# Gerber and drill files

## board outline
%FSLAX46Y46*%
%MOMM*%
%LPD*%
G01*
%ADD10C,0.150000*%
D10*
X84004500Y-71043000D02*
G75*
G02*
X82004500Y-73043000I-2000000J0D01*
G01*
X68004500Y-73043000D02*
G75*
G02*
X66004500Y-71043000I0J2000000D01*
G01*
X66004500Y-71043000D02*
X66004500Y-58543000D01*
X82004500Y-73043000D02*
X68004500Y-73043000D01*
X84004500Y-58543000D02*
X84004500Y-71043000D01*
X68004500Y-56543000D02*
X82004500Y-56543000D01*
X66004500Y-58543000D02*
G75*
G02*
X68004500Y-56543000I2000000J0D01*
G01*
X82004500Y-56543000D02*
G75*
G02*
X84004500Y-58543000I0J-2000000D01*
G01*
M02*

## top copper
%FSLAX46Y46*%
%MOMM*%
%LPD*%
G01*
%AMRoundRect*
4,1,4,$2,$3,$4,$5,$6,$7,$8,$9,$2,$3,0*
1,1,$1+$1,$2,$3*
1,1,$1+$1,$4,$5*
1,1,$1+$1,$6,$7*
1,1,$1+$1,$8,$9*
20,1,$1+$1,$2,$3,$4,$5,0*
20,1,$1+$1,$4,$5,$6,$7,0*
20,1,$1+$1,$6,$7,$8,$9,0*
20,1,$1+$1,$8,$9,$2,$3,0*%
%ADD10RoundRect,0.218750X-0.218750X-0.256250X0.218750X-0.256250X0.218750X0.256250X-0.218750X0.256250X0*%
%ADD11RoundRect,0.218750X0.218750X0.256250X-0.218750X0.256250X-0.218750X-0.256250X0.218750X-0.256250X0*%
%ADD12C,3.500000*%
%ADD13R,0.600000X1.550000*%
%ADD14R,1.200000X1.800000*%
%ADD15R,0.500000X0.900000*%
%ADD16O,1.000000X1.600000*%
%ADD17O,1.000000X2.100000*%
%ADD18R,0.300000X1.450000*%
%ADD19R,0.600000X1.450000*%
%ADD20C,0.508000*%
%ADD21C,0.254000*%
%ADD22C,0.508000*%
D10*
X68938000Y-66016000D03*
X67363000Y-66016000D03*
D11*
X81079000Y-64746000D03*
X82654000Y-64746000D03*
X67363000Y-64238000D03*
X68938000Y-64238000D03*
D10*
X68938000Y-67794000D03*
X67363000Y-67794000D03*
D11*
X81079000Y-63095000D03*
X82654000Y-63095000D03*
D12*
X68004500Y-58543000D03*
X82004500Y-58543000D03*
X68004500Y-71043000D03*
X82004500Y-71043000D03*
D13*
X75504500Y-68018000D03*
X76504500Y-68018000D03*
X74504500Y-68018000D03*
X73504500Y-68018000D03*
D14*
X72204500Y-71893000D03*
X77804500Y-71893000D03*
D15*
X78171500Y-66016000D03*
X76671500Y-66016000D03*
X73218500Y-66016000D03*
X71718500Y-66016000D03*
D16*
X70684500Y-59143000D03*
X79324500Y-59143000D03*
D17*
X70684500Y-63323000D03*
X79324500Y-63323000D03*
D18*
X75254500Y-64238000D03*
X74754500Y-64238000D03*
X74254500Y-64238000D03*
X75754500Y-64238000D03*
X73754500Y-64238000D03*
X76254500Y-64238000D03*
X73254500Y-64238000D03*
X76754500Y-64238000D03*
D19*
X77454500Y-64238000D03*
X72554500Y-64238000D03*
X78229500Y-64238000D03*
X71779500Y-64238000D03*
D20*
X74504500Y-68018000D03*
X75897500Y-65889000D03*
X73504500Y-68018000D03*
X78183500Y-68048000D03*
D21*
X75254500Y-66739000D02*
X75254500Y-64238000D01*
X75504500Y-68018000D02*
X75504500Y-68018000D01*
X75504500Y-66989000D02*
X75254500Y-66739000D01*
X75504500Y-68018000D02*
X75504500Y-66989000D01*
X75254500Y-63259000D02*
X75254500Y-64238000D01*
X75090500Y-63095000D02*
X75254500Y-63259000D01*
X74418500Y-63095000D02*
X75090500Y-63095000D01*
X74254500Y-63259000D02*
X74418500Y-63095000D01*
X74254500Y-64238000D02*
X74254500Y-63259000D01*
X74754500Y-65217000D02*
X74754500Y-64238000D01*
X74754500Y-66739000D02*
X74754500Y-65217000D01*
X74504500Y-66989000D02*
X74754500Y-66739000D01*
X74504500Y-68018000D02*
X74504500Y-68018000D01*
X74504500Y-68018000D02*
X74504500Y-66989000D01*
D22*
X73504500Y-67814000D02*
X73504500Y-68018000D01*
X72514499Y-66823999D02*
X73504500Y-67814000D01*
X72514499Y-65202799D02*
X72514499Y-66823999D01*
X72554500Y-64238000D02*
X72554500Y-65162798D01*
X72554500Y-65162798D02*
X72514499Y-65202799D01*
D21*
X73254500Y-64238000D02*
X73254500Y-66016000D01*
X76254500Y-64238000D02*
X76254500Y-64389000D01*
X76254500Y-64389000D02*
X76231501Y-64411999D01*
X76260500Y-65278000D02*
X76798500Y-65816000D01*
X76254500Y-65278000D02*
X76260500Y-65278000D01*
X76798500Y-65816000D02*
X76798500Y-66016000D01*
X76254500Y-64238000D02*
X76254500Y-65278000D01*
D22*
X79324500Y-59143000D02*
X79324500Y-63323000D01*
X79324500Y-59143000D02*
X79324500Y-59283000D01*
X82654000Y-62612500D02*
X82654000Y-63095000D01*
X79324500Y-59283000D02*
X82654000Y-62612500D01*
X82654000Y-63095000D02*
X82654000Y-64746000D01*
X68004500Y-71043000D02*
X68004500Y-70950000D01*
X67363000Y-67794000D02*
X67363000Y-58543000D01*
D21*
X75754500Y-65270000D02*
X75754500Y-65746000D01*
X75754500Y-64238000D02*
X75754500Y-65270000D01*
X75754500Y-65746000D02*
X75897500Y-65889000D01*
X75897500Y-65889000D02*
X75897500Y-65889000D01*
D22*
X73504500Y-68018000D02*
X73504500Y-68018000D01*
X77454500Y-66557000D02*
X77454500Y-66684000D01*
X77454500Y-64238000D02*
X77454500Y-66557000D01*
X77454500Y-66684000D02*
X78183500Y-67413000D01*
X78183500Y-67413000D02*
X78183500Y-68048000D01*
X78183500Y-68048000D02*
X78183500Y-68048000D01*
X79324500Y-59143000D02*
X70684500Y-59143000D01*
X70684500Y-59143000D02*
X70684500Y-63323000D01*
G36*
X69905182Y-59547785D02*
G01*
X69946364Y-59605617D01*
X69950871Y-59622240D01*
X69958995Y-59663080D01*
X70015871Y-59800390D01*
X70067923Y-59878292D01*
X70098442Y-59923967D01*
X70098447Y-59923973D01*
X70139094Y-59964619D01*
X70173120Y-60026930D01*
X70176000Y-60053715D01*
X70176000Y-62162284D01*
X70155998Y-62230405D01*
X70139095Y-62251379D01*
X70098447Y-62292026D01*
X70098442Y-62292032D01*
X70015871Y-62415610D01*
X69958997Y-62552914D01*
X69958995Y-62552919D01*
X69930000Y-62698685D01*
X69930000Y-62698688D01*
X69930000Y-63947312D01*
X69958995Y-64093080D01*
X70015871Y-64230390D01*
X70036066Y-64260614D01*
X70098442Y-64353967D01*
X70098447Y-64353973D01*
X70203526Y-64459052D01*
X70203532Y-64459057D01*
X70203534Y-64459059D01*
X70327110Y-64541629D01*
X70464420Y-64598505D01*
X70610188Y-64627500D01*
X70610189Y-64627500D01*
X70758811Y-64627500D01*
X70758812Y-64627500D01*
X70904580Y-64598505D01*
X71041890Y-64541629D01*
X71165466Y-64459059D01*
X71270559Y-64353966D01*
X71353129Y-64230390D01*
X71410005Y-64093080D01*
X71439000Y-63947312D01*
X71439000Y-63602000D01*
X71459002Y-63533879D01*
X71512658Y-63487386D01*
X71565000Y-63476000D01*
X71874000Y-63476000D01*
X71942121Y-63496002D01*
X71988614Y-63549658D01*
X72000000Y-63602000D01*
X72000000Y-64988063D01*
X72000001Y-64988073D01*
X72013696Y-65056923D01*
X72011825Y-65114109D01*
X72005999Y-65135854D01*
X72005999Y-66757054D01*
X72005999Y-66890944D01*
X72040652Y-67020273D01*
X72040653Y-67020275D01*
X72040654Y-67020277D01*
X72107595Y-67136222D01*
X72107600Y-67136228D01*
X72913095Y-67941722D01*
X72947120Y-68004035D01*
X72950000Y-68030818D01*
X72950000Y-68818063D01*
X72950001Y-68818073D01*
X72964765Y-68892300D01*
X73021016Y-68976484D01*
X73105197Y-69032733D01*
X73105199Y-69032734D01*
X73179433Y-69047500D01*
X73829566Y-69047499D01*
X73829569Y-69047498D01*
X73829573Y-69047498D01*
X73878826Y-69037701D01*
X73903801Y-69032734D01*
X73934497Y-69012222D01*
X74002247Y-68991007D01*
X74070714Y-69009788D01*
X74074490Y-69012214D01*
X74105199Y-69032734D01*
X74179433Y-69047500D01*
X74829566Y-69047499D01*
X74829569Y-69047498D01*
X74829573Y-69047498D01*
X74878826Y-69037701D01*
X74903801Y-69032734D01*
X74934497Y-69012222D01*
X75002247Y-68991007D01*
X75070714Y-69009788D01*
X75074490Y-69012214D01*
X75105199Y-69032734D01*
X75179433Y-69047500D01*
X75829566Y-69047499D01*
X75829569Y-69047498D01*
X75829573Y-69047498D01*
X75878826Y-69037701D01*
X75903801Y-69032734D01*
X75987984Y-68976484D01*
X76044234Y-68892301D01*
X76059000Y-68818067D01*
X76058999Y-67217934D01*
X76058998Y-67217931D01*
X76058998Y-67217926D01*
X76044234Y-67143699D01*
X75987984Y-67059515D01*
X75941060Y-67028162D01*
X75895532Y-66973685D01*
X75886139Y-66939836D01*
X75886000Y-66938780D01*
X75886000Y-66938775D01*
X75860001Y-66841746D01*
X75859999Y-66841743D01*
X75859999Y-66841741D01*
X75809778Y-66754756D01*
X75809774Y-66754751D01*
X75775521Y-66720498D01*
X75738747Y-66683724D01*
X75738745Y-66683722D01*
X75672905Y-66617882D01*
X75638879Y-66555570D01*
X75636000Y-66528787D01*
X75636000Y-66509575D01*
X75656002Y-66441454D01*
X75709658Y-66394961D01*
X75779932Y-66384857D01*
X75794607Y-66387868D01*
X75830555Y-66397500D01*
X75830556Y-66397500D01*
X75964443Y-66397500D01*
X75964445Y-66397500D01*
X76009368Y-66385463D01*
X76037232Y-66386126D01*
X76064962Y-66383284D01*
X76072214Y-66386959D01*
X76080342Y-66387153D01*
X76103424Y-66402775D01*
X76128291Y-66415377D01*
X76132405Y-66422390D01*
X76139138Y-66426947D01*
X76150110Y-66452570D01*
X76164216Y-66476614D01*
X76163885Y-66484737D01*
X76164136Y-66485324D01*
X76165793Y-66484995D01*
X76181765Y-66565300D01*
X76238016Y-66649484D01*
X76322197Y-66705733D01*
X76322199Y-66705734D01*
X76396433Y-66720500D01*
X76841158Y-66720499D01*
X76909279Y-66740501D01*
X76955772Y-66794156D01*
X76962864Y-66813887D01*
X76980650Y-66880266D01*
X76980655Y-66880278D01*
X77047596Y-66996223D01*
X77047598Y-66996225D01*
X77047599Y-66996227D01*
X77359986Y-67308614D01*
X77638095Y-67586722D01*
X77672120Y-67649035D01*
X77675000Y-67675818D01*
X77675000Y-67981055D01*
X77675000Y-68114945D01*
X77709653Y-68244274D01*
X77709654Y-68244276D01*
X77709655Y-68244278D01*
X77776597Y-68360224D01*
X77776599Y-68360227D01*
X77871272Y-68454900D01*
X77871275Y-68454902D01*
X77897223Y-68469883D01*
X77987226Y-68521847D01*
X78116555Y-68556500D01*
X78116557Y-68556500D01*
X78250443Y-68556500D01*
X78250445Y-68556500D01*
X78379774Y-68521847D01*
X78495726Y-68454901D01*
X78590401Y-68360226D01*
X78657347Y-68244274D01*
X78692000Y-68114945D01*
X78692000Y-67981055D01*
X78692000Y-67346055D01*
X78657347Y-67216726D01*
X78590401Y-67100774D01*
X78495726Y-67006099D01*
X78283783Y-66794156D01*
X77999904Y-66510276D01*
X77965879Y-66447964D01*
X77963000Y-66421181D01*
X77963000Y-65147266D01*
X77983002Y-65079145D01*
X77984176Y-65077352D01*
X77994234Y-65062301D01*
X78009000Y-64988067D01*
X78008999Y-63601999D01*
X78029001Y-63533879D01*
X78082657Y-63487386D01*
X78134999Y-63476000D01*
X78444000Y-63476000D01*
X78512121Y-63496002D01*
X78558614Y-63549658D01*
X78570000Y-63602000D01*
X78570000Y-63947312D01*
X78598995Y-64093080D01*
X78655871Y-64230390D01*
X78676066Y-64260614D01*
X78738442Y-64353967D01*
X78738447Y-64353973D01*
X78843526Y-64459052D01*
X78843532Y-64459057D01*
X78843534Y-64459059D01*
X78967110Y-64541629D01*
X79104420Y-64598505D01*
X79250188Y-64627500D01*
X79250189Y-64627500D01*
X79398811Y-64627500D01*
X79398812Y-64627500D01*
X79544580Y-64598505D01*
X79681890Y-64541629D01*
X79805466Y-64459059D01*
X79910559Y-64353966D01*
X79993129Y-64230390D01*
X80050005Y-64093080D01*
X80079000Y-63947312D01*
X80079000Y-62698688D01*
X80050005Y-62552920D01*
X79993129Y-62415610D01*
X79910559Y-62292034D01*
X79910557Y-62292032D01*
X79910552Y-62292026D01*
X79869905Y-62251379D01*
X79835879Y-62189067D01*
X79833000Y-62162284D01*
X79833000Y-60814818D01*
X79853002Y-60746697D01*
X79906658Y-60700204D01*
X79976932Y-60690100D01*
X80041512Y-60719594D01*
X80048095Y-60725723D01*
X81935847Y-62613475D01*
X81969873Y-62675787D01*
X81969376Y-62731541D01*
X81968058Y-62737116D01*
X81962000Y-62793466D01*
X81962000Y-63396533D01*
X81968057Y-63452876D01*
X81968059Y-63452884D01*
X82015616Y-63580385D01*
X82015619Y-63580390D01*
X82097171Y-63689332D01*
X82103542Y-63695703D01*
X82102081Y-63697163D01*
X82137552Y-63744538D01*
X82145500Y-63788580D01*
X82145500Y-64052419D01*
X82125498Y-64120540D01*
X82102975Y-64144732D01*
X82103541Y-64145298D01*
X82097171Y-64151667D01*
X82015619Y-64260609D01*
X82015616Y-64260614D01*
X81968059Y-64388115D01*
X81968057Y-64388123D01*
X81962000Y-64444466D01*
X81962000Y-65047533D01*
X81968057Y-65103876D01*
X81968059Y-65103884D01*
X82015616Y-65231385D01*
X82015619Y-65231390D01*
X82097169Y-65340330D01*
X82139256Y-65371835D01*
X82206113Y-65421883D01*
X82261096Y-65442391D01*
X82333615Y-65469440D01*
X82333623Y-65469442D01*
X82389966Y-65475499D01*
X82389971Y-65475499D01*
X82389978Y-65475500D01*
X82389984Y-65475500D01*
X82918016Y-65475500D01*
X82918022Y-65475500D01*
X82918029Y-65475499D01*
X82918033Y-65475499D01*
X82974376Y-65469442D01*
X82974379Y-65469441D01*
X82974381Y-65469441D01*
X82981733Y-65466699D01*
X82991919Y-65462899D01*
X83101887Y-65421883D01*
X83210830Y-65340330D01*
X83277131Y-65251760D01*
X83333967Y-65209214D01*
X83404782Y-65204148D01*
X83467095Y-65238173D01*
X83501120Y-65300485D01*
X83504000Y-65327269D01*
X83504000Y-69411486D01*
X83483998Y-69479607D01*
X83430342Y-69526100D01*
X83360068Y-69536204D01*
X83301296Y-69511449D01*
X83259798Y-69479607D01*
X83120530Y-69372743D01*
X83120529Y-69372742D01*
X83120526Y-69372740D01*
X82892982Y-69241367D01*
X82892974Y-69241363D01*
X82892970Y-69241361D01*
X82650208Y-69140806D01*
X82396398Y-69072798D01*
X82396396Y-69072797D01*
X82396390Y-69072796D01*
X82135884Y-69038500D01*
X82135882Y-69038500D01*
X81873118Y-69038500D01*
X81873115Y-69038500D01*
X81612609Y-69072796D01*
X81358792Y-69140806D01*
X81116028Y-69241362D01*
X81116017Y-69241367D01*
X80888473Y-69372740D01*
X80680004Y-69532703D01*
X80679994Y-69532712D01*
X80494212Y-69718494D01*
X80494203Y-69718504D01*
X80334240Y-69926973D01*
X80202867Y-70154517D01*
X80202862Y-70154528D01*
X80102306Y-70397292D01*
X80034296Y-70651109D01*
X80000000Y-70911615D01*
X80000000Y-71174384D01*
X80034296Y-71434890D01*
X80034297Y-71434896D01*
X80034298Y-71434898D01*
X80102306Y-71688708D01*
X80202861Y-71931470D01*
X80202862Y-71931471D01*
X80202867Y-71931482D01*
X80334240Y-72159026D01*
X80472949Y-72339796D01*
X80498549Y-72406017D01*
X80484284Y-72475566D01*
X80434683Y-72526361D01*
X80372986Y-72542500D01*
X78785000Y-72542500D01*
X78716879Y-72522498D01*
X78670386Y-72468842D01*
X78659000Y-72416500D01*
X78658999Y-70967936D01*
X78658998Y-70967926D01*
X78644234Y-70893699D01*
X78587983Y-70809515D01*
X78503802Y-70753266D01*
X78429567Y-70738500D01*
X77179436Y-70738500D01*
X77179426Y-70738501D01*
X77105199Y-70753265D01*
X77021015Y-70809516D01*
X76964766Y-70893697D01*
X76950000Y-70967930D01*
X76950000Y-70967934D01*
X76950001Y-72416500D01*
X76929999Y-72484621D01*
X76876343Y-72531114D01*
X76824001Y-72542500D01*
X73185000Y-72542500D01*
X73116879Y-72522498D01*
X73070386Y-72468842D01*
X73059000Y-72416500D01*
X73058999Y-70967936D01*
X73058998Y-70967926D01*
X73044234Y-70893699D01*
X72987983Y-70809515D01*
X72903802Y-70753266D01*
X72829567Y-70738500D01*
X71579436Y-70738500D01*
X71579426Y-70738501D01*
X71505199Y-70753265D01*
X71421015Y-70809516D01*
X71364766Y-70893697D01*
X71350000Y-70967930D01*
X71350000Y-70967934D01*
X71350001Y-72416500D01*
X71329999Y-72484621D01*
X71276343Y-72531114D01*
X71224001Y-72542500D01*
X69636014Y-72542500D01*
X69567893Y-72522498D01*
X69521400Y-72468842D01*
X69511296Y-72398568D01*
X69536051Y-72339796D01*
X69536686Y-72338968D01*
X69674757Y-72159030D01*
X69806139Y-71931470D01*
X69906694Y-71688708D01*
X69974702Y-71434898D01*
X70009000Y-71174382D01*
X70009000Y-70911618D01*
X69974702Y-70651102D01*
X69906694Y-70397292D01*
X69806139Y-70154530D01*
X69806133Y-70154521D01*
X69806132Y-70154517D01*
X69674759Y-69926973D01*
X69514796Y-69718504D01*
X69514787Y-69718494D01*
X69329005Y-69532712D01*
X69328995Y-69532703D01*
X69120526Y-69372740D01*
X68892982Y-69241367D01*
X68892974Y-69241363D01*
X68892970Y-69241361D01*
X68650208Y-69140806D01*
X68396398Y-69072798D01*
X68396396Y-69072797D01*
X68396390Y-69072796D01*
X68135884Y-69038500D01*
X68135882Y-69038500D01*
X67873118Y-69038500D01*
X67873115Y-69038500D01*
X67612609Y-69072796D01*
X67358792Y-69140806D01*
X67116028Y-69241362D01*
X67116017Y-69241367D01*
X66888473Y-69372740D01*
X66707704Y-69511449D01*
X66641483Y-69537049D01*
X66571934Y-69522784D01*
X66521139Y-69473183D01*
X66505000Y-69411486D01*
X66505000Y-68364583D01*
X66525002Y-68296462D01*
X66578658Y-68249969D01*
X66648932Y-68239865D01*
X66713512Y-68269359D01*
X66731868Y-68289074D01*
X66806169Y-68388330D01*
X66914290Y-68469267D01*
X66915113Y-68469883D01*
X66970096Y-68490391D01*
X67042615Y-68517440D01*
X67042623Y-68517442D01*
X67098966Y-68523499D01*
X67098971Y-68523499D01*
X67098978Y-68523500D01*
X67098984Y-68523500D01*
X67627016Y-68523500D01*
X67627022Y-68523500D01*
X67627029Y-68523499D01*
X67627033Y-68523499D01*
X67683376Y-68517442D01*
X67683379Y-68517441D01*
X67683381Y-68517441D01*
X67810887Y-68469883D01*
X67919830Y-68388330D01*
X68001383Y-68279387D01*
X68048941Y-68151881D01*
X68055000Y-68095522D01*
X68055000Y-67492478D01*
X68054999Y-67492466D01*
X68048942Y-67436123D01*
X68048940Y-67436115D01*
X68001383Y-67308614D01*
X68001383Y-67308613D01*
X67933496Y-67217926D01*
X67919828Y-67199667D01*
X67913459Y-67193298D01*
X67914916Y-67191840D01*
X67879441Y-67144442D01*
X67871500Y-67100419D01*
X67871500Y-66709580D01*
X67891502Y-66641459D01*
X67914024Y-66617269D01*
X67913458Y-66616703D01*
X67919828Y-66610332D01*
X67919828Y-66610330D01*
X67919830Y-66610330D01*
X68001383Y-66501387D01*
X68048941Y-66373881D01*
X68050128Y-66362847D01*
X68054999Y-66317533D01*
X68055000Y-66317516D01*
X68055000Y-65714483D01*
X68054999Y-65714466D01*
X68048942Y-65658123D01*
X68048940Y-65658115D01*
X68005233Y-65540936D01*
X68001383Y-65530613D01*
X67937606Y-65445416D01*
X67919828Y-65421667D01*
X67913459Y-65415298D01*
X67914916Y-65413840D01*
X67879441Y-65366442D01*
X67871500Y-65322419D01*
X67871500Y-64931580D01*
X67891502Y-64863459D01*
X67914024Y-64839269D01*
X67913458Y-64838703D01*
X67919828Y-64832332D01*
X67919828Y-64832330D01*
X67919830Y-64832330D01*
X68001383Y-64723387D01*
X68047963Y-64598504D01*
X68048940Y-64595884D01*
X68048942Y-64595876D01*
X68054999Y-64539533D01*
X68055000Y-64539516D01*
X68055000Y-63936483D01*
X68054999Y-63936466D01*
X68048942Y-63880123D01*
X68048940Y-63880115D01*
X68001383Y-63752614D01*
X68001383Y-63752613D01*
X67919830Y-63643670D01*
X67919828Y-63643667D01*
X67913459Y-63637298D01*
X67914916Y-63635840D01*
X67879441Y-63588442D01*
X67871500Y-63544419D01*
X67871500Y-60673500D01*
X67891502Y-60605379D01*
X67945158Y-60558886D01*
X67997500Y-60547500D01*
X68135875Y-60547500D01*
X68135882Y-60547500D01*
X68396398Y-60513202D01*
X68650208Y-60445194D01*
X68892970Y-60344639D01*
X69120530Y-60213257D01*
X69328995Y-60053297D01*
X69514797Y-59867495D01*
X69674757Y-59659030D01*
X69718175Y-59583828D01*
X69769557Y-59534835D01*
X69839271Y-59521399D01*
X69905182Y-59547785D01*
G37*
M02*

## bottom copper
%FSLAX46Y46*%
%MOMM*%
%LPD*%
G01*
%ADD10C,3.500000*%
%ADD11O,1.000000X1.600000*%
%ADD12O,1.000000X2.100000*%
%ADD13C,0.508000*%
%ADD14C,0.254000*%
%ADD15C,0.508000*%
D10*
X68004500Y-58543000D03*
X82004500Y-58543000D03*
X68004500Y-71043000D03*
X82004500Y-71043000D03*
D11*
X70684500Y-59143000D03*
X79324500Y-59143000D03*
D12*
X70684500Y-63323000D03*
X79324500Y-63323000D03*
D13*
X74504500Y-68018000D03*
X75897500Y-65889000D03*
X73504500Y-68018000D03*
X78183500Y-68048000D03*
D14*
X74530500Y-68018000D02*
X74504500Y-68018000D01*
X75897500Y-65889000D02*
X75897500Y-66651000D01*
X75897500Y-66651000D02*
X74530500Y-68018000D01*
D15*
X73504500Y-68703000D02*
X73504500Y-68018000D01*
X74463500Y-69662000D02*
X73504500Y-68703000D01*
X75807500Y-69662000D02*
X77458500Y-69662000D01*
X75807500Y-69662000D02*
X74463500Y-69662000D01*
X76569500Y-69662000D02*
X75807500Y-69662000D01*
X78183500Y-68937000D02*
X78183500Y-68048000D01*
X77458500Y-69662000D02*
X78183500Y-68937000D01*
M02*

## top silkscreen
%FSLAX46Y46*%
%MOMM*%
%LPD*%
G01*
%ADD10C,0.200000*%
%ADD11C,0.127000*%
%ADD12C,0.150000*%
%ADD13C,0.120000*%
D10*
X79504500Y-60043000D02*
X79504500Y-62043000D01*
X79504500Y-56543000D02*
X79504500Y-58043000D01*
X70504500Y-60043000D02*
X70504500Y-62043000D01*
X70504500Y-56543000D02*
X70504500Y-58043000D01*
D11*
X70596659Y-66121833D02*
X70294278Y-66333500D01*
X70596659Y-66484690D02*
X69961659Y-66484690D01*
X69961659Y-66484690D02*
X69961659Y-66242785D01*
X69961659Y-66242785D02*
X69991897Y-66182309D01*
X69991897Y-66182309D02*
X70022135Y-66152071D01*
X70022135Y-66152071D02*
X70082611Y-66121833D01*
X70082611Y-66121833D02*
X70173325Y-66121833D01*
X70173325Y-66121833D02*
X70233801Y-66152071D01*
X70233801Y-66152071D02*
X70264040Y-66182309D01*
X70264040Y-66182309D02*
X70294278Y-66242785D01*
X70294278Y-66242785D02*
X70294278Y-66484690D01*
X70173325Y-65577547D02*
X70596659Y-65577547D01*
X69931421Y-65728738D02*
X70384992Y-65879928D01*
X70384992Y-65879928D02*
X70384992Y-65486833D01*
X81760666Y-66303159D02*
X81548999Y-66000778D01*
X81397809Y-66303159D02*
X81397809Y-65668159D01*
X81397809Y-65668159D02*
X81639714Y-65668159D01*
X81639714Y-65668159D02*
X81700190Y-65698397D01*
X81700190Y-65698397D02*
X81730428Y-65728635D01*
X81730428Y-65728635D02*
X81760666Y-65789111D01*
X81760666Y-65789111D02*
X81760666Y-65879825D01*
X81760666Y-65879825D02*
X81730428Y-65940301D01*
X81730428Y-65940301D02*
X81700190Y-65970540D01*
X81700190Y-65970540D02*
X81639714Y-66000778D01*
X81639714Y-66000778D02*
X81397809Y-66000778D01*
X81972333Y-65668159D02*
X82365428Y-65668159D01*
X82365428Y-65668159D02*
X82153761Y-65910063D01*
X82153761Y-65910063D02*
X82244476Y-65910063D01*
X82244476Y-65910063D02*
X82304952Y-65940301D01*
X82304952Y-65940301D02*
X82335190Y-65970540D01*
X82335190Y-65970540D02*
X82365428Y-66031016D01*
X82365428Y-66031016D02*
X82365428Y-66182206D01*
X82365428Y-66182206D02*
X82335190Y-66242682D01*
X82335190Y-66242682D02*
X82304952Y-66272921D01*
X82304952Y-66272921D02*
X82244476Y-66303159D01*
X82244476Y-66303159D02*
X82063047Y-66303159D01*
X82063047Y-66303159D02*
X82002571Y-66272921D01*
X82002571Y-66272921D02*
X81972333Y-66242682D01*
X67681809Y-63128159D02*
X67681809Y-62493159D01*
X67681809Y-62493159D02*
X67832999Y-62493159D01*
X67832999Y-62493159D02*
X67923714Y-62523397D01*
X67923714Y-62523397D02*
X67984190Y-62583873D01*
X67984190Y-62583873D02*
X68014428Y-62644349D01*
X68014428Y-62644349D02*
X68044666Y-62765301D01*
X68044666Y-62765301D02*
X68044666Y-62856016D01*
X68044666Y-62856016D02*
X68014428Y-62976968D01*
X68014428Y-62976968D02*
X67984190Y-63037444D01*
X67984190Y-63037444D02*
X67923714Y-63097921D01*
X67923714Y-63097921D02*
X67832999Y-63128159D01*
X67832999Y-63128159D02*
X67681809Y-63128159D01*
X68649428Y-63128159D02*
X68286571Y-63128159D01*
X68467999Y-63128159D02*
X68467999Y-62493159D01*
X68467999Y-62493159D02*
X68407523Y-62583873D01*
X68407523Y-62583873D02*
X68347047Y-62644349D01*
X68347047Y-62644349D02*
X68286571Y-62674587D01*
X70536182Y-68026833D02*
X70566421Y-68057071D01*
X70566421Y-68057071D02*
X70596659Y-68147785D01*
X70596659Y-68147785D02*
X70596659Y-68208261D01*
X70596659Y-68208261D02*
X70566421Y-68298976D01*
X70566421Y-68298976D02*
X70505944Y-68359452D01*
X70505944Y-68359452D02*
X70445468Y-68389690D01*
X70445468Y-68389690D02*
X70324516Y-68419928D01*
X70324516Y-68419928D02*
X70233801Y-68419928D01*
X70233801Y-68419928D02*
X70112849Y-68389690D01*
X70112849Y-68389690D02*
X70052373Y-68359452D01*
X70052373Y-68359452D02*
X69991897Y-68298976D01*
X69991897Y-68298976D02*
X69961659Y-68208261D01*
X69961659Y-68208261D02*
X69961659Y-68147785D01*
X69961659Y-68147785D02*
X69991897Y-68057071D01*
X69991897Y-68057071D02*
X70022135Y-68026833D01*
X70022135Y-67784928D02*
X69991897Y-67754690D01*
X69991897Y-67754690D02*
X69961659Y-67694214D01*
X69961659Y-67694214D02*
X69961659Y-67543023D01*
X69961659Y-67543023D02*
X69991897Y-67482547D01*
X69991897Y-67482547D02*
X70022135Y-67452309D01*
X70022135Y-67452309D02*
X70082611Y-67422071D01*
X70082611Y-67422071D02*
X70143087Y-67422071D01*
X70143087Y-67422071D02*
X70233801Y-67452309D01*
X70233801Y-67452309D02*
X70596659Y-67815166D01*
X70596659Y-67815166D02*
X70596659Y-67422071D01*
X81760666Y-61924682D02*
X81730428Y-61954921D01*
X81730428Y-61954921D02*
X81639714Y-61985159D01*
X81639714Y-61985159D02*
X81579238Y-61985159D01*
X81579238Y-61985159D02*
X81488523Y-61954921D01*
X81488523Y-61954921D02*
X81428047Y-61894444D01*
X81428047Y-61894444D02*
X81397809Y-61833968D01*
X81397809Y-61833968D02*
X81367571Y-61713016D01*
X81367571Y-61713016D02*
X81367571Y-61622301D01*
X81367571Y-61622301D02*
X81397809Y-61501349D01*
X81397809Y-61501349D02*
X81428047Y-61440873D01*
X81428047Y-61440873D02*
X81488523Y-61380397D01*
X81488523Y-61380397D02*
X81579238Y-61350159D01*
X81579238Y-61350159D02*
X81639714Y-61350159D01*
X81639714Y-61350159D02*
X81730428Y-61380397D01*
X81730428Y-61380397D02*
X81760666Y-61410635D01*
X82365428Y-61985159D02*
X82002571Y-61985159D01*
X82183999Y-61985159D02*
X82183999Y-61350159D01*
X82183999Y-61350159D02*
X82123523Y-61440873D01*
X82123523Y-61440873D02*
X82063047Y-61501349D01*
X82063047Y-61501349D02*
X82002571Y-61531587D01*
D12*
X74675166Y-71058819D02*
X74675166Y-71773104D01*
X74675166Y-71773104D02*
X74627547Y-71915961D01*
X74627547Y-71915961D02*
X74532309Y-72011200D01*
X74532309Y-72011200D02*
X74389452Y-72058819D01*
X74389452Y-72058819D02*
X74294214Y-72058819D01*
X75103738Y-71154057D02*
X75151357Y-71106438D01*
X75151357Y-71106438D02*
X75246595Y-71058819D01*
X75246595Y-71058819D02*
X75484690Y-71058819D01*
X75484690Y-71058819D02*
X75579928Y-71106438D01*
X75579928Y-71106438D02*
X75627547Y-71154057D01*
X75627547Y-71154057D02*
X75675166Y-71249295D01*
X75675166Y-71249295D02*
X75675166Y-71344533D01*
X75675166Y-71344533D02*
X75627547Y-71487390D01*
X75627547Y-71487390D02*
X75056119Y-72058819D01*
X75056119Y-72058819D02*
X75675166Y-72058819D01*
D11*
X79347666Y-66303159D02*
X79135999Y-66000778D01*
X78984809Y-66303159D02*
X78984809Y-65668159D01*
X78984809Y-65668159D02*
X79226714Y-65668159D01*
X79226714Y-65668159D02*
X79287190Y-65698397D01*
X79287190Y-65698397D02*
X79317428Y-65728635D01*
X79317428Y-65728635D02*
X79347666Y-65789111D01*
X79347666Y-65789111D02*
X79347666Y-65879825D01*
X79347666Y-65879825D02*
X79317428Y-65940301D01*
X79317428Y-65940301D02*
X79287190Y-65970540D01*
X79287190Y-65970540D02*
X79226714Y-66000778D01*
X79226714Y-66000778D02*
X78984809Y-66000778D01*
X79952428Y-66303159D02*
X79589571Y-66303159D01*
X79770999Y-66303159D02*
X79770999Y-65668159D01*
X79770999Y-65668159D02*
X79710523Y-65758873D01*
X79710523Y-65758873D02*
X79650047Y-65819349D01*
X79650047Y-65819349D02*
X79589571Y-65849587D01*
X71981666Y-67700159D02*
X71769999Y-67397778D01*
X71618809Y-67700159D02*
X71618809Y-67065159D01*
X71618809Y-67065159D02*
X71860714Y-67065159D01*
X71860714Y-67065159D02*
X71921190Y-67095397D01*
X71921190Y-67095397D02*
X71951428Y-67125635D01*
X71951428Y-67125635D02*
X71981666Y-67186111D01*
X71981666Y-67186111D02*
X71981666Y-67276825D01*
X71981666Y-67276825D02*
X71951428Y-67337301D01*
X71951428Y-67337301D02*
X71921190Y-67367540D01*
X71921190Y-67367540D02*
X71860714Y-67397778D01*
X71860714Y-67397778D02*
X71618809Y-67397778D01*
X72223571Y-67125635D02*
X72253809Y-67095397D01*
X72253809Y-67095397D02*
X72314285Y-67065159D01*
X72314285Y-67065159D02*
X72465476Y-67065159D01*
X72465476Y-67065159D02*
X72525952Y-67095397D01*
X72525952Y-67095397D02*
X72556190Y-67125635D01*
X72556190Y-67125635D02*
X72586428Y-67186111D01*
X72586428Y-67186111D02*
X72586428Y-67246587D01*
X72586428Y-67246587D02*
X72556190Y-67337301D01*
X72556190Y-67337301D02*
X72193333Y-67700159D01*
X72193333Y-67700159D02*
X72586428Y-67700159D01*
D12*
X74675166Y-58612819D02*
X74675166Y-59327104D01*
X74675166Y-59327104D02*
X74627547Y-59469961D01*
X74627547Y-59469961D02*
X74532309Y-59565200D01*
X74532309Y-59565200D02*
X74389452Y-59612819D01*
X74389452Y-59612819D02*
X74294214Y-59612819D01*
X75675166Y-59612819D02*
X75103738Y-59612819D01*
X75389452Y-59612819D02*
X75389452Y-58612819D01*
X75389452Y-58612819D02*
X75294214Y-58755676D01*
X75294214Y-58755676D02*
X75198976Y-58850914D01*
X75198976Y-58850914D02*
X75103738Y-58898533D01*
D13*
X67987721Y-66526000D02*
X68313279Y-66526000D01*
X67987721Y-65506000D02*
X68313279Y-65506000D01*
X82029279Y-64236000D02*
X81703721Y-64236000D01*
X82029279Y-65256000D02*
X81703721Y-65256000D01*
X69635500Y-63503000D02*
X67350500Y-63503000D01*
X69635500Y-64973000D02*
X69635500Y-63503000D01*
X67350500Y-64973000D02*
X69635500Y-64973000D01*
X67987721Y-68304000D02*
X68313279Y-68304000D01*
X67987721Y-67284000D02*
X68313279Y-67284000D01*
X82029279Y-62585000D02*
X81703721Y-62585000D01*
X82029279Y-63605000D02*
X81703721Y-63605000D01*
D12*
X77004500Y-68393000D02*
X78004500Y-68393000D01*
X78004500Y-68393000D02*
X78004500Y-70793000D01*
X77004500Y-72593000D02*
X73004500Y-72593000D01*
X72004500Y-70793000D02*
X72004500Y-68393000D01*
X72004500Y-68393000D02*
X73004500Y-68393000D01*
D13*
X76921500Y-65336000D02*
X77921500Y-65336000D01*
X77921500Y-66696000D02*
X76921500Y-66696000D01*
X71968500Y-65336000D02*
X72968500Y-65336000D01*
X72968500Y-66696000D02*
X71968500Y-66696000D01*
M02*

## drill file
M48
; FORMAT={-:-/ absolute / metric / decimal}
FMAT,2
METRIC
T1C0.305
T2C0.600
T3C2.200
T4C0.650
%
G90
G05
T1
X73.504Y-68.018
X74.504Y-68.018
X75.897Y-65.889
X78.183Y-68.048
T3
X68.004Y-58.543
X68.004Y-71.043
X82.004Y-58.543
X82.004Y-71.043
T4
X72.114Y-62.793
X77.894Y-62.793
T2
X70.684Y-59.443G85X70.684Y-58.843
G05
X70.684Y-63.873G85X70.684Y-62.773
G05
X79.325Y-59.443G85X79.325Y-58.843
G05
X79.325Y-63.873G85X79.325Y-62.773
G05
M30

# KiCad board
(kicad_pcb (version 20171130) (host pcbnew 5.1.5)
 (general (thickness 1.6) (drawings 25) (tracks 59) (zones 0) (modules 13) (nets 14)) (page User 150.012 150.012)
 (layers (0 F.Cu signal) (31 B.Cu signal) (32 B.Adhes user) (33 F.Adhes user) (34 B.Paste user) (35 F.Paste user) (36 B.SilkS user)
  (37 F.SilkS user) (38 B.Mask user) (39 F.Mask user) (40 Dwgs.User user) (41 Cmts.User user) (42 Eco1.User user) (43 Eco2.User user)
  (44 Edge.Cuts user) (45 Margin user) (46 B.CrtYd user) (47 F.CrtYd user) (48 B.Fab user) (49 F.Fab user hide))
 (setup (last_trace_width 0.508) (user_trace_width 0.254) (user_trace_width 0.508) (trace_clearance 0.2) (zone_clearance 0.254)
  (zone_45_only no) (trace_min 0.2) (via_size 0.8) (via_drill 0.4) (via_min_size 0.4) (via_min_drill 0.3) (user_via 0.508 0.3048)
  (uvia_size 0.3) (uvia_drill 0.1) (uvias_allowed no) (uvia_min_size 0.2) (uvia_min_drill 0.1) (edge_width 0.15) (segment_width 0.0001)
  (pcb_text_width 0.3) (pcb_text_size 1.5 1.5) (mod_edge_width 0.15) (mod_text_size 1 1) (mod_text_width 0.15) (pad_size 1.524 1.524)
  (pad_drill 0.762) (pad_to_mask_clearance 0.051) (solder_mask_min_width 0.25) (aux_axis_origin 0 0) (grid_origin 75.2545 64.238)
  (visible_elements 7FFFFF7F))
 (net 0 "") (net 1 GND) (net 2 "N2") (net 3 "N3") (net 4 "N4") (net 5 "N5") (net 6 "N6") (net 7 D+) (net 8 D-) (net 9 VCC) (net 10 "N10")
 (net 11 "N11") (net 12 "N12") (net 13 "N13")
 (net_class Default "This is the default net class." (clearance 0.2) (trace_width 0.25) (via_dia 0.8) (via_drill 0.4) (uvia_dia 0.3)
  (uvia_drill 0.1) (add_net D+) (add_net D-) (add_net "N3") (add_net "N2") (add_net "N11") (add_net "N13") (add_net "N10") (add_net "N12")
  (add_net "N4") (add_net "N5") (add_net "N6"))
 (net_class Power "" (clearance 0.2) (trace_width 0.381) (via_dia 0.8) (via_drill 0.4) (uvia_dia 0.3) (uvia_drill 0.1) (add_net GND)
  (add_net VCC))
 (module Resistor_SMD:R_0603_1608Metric (layer F.Cu) (at 68.1505 66.016)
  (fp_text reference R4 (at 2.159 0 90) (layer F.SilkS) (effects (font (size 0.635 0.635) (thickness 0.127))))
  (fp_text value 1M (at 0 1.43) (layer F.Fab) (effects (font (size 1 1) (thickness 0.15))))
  (fp_line (start -0.162779 0.51) (end 0.162779 0.51) (layer F.SilkS) (width 0.12))
  (fp_line (start -0.162779 -0.51) (end 0.162779 -0.51) (layer F.SilkS) (width 0.12))
  (pad 2 smd roundrect (at 0.7875 0) (size 0.875 0.95) (layers F.Cu F.Paste F.Mask) (roundrect_rratio 0.25) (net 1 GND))
  (pad 1 smd roundrect (at -0.7875 0) (size 0.875 0.95) (layers F.Cu F.Paste F.Mask) (roundrect_rratio 0.25) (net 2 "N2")))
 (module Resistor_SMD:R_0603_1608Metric (layer F.Cu) (at 81.8665 64.746 180)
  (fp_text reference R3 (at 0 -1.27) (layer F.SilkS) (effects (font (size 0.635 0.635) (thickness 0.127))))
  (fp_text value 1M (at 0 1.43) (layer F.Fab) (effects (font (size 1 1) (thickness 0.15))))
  (fp_line (start -0.162779 0.51) (end 0.162779 0.51) (layer F.SilkS) (width 0.12))
  (fp_line (start -0.162779 -0.51) (end 0.162779 -0.51) (layer F.SilkS) (width 0.12))
  (pad 2 smd roundrect (at 0.7875 0 180) (size 0.875 0.95) (layers F.Cu F.Paste F.Mask) (roundrect_rratio 0.25) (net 1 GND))
  (pad 1 smd roundrect (at -0.7875 0 180) (size 0.875 0.95) (layers F.Cu F.Paste F.Mask) (roundrect_rratio 0.25) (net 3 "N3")))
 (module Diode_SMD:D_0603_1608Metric (layer F.Cu) (at 68.1505 64.238 180)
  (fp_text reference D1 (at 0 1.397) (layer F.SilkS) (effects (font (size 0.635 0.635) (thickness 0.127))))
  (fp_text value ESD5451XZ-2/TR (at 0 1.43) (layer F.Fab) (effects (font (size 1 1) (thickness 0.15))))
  (fp_line (start -1.485 0.735) (end 0.8 0.735) (layer F.SilkS) (width 0.12))
  (fp_line (start -1.485 -0.735) (end -1.485 0.735) (layer F.SilkS) (width 0.12))
  (fp_line (start 0.8 -0.735) (end -1.485 -0.735) (layer F.SilkS) (width 0.12))
  (pad 2 smd roundrect (at 0.7875 0 180) (size 0.875 0.95) (layers F.Cu F.Paste F.Mask) (roundrect_rratio 0.25) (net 2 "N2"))
  (pad 1 smd roundrect (at -0.7875 0 180) (size 0.875 0.95) (layers F.Cu F.Paste F.Mask) (roundrect_rratio 0.25) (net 1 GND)))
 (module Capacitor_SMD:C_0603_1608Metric (layer F.Cu) (at 68.1505 67.794)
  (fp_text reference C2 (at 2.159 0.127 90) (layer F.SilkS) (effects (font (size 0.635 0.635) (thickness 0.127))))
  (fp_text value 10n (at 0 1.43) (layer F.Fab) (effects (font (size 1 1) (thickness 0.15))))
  (fp_line (start -0.162779 0.51) (end 0.162779 0.51) (layer F.SilkS) (width 0.12))
  (fp_line (start -0.162779 -0.51) (end 0.162779 -0.51) (layer F.SilkS) (width 0.12))
  (pad 2 smd roundrect (at 0.7875 0) (size 0.875 0.95) (layers F.Cu F.Paste F.Mask) (roundrect_rratio 0.25) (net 1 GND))
  (pad 1 smd roundrect (at -0.7875 0) (size 0.875 0.95) (layers F.Cu F.Paste F.Mask) (roundrect_rratio 0.25) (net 2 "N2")))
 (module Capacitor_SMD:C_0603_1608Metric (layer F.Cu) (at 81.8665 63.095 180)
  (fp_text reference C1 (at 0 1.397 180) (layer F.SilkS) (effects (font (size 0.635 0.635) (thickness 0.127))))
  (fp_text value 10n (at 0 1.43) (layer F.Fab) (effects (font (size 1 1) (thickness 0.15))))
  (fp_line (start -0.162779 0.51) (end 0.162779 0.51) (layer F.SilkS) (width 0.12))
  (fp_line (start -0.162779 -0.51) (end 0.162779 -0.51) (layer F.SilkS) (width 0.12))
  (pad 2 smd roundrect (at 0.7875 0 180) (size 0.875 0.95) (layers F.Cu F.Paste F.Mask) (roundrect_rratio 0.25) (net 1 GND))
  (pad 1 smd roundrect (at -0.7875 0 180) (size 0.875 0.95) (layers F.Cu F.Paste F.Mask) (roundrect_rratio 0.25) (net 3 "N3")))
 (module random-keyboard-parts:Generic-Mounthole (layer F.Cu) (at 68.0045 58.543)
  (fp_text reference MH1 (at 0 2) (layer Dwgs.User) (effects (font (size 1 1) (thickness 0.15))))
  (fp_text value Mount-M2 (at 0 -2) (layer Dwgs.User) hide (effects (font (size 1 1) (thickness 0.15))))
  (pad 1 thru_hole circle (at 0 0) (size 3.5 3.5) (drill 2.2) (layers *.Cu *.Mask) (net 2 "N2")))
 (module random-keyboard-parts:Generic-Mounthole (layer F.Cu) (at 82.0045 58.543)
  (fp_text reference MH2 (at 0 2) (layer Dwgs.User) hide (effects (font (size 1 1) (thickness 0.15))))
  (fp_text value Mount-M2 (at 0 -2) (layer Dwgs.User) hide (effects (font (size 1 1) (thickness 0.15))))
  (pad 1 thru_hole circle (at 0 0) (size 3.5 3.5) (drill 2.2) (layers *.Cu *.Mask) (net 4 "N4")))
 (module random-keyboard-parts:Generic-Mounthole (layer F.Cu) (at 68.0045 71.043)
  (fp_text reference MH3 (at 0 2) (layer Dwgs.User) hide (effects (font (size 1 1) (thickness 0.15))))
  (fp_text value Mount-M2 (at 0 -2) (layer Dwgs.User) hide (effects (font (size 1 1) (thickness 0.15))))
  (pad 1 thru_hole circle (at 0 0) (size 3.5 3.5) (drill 2.2) (layers *.Cu *.Mask) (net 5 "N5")))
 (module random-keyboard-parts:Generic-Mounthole (layer F.Cu) (at 82.0045 71.043)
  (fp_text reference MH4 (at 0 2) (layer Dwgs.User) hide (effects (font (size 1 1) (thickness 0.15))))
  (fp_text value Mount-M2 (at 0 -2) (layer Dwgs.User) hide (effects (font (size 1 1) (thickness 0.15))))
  (pad 1 thru_hole circle (at 0 0) (size 3.5 3.5) (drill 2.2) (layers *.Cu *.Mask) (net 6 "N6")))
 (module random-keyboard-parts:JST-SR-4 (layer F.Cu) (at 75.0045 72.793)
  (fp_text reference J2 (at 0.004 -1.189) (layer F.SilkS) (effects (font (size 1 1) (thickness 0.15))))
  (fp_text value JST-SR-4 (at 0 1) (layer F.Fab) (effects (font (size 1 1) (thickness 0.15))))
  (fp_line (start 2 -4.4) (end 3 -4.4) (layer F.SilkS) (width 0.15))
  (fp_line (start 3 -4.4) (end 3 -2) (layer F.SilkS) (width 0.15))
  (fp_line (start 2 -0.2) (end -2 -0.2) (layer F.SilkS) (width 0.15))
  (fp_line (start -3 -2) (end -3 -4.4) (layer F.SilkS) (width 0.15))
  (fp_line (start -3 -4.4) (end -2 -4.4) (layer F.SilkS) (width 0.15))
  (pad 3 smd rect (at 0.5 -4.775) (size 0.6 1.55) (layers F.Cu F.Paste F.Mask) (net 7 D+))
  (pad 4 smd rect (at 1.5 -4.775) (size 0.6 1.55) (layers F.Cu F.Paste F.Mask) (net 1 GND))
  (pad 2 smd rect (at -0.5 -4.775) (size 0.6 1.55) (layers F.Cu F.Paste F.Mask) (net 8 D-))
  (pad 1 smd rect (at -1.5 -4.775) (size 0.6 1.55) (layers F.Cu F.Paste F.Mask) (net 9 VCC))
  (pad "" smd rect (at -2.8 -0.9) (size 1.2 1.8) (layers F.Cu F.Paste F.Mask))
  (pad "" smd rect (at 2.8 -0.9) (size 1.2 1.8) (layers F.Cu F.Paste F.Mask)))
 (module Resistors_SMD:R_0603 (layer F.Cu) (at 77.4215 66.016)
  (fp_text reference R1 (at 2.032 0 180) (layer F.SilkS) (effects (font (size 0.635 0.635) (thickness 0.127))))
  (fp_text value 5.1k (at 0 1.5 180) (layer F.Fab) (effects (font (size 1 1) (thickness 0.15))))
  (fp_line (start -0.5 -0.68) (end 0.5 -0.68) (layer F.SilkS) (width 0.12))
  (fp_line (start 0.5 0.68) (end -0.5 0.68) (layer F.SilkS) (width 0.12))
  (pad 2 smd rect (at 0.75 0) (size 0.5 0.9) (layers F.Cu F.Paste F.Mask) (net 1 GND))
  (pad 1 smd rect (at -0.75 0) (size 0.5 0.9) (layers F.Cu F.Paste F.Mask) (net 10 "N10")))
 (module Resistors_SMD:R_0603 (layer F.Cu) (at 72.4685 66.016 180)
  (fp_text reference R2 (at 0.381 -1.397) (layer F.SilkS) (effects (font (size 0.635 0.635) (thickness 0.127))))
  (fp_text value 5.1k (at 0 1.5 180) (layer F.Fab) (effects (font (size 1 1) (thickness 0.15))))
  (fp_line (start 0.5 0.68) (end -0.5 0.68) (layer F.SilkS) (width 0.12))
  (fp_line (start -0.5 -0.68) (end 0.5 -0.68) (layer F.SilkS) (width 0.12))
  (pad 1 smd rect (at -0.75 0 180) (size 0.5 0.9) (layers F.Cu F.Paste F.Mask) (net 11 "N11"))
  (pad 2 smd rect (at 0.75 0 180) (size 0.5 0.9) (layers F.Cu F.Paste F.Mask) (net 1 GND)))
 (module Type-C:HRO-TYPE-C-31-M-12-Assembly (layer F.Cu) (at 75.0045 56.543 180)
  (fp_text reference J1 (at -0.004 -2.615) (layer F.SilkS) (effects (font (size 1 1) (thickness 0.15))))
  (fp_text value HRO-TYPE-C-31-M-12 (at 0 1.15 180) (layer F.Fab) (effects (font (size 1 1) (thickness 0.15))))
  (pad 13 thru_hole oval (at 4.32 -2.6 180) (size 1 1.6) (drill oval 0.6 1.2) (layers *.Cu *.Mask) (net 3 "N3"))
  (pad 13 thru_hole oval (at -4.32 -2.6 180) (size 1 1.6) (drill oval 0.6 1.2) (layers *.Cu *.Mask) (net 3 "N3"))
  (pad 13 thru_hole oval (at 4.32 -6.78 180) (size 1 2.1) (drill oval 0.6 1.7) (layers *.Cu *.Mask) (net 3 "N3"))
  (pad 13 thru_hole oval (at -4.32 -6.78 180) (size 1 2.1) (drill oval 0.6 1.7) (layers *.Cu *.Mask) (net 3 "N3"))
  (pad "" np_thru_hole circle (at -2.89 -6.25 180) (size 0.65 0.65) (drill 0.65) (layers *.Cu *.Mask))
  (pad "" np_thru_hole circle (at 2.89 -6.25 180) (size 0.65 0.65) (drill 0.65) (layers *.Cu *.Mask))
  (pad 6 smd rect (at -0.25 -7.695 180) (size 0.3 1.45) (layers F.Cu F.Paste F.Mask) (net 7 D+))
  (pad 7 smd rect (at 0.25 -7.695 180) (size 0.3 1.45) (layers F.Cu F.Paste F.Mask) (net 8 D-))
  (pad 8 smd rect (at 0.75 -7.695 180) (size 0.3 1.45) (layers F.Cu F.Paste F.Mask) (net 7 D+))
  (pad 5 smd rect (at -0.75 -7.695 180) (size 0.3 1.45) (layers F.Cu F.Paste F.Mask) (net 8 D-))
  (pad 9 smd rect (at 1.25 -7.695 180) (size 0.3 1.45) (layers F.Cu F.Paste F.Mask) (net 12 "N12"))
  (pad 4 smd rect (at -1.25 -7.695 180) (size 0.3 1.45) (layers F.Cu F.Paste F.Mask) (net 10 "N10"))
  (pad 10 smd rect (at 1.75 -7.695 180) (size 0.3 1.45) (layers F.Cu F.Paste F.Mask) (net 11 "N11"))
  (pad 3 smd rect (at -1.75 -7.695 180) (size 0.3 1.45) (layers F.Cu F.Paste F.Mask) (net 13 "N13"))
  (pad 2 smd rect (at -2.45 -7.695 180) (size 0.6 1.45) (layers F.Cu F.Paste F.Mask) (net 9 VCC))
  (pad 11 smd rect (at 2.45 -7.695 180) (size 0.6 1.45) (layers F.Cu F.Paste F.Mask) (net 9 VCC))
  (pad 1 smd rect (at -3.225 -7.695 180) (size 0.6 1.45) (layers F.Cu F.Paste F.Mask) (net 1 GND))
  (pad 12 smd rect (at 3.225 -7.695 180) (size 0.6 1.45) (layers F.Cu F.Paste F.Mask) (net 1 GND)))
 (gr_line (start 79.5045 60.043) (end 79.5045 62.043) (layer F.SilkS) (width 0.2))
 (gr_line (start 79.5045 56.543) (end 79.5045 58.043) (layer F.SilkS) (width 0.2))
 (gr_line (start 70.5045 60.043) (end 70.5045 62.043) (layer F.SilkS) (width 0.2))
 (gr_line (start 70.5045 56.543) (end 70.5045 58.043) (layer F.SilkS) (width 0.2))
 (gr_arc (start 82.0045 71.043) (end 82.0045 73.043) (angle -90) (layer Edge.Cuts) (width 0.15))
 (gr_arc (start 68.0045 71.043) (end 66.0045 71.043) (angle -90) (layer Edge.Cuts) (width 0.15))
 (gr_line (start 66.0045 71.043) (end 66.0045 58.543) (layer Edge.Cuts) (width 0.15))
 (gr_line (start 82.0045 73.043) (end 68.0045 73.043) (layer Edge.Cuts) (width 0.15))
 (gr_line (start 84.0045 58.543) (end 84.0045 71.043) (layer Edge.Cuts) (width 0.15))
 (gr_line (start 68.0045 56.543) (end 82.0045 56.543) (layer Edge.Cuts) (width 0.15))
 (gr_arc (start 68.0045 58.543) (end 68.0045 56.543) (angle -90) (layer Edge.Cuts) (width 0.15))
 (gr_arc (start 82.0045 58.543) (end 84.0045 58.543) (angle -90) (layer Edge.Cuts) (width 0.15))
 (segment (start 75.2545 66.739) (end 75.2545 64.238) (width 0.254) (layer F.Cu) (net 7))
 (segment (start 75.5045 68.018) (end 75.5045 68.018) (width 0.254) (layer F.Cu) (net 7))
 (segment (start 75.5045 66.989) (end 75.2545 66.739) (width 0.254) (layer F.Cu) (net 7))
 (segment (start 75.5045 68.018) (end 75.5045 66.989) (width 0.254) (layer F.Cu) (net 7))
 (segment (start 75.2545 63.259) (end 75.2545 64.238) (width 0.254) (layer F.Cu) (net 7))
 (segment (start 75.0905 63.095) (end 75.2545 63.259) (width 0.254) (layer F.Cu) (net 7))
 (segment (start 74.4185 63.095) (end 75.0905 63.095) (width 0.254) (layer F.Cu) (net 7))
 (segment (start 74.2545 63.259) (end 74.4185 63.095) (width 0.254) (layer F.Cu) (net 7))
 (segment (start 74.2545 64.238) (end 74.2545 63.259) (width 0.254) (layer F.Cu) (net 7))
 (segment (start 74.7545 65.217) (end 74.7545 64.238) (width 0.254) (layer F.Cu) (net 8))
 (segment (start 74.7545 66.739) (end 74.7545 65.217) (width 0.254) (layer F.Cu) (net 8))
 (segment (start 74.5045 66.989) (end 74.7545 66.739) (width 0.254) (layer F.Cu) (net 8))
 (segment (start 74.5045 68.018) (end 74.5045 68.018) (width 0.254) (layer F.Cu) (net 8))
 (segment (start 74.5045 68.018) (end 74.5045 66.989) (width 0.254) (layer F.Cu) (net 8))
 (via (at 74.5045 68.018) (size 0.508) (drill 0.3048) (layers F.Cu B.Cu) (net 8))
 (segment (start 73.5045 67.814) (end 73.5045 68.018) (width 0.508) (layer F.Cu) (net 9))
 (segment (start 72.514499 66.823999) (end 73.5045 67.814) (width 0.508) (layer F.Cu) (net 9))
 (segment (start 72.514499 65.202799) (end 72.514499 66.823999) (width 0.508) (layer F.Cu) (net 9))
 (segment (start 72.5545 64.238) (end 72.5545 65.162798) (width 0.508) (layer F.Cu) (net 9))
 (segment (start 72.5545 65.162798) (end 72.514499 65.202799) (width 0.508) (layer F.Cu) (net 9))
 (segment (start 73.2545 64.238) (end 73.2545 66.016) (width 0.254) (layer F.Cu) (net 11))
 (segment (start 76.2545 64.238) (end 76.2545 64.389) (width 0.254) (layer F.Cu) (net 10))
 (segment (start 76.2545 64.389) (end 76.231501 64.411999) (width 0.254) (layer F.Cu) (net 10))
 (segment (start 76.2605 65.278) (end 76.7985 65.816) (width 0.254) (layer F.Cu) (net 10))
 (segment (start 76.2545 65.278) (end 76.2605 65.278) (width 0.254) (layer F.Cu) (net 10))
 (segment (start 76.7985 65.816) (end 76.7985 66.016) (width 0.254) (layer F.Cu) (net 10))
 (segment (start 76.2545 64.238) (end 76.2545 65.278) (width 0.254) (layer F.Cu) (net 10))
 (segment (start 79.3245 59.143) (end 79.3245 63.323) (width 0.508) (layer F.Cu) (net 3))
 (segment (start 79.3245 59.143) (end 79.3245 59.283) (width 0.508) (layer F.Cu) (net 3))
 (segment (start 82.654 62.6125) (end 82.654 63.095) (width 0.508) (layer F.Cu) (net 3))
 (segment (start 79.3245 59.283) (end 82.654 62.6125) (width 0.508) (layer F.Cu) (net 3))
 (segment (start 82.654 63.095) (end 82.654 64.746) (width 0.508) (layer F.Cu) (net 3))
 (segment (start 68.0045 71.043) (end 68.0045 70.95) (width 0.508) (layer F.Cu) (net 5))
 (segment (start 67.363 67.794) (end 67.363 58.543) (width 0.508) (layer F.Cu) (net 2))
 (segment (start 75.7545 65.27) (end 75.7545 65.746) (width 0.254) (layer F.Cu) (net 8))
 (segment (start 75.7545 64.238) (end 75.7545 65.27) (width 0.254) (layer F.Cu) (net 8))
 (segment (start 75.7545 65.746) (end 75.8975 65.889) (width 0.254) (layer F.Cu) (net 8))
 (segment (start 75.8975 65.889) (end 75.8975 65.889) (width 0.254) (layer F.Cu) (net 8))
 (via (at 75.8975 65.889) (size 0.508) (drill 0.3048) (layers F.Cu B.Cu) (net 8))
 (segment (start 74.5305 68.018) (end 74.5045 68.018) (width 0.254) (layer B.Cu) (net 8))
 (segment (start 75.8975 65.889) (end 75.8975 66.651) (width 0.254) (layer B.Cu) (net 8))
 (segment (start 75.8975 66.651) (end 74.5305 68.018) (width 0.254) (layer B.Cu) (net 8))
 (segment (start 73.5045 68.018) (end 73.5045 68.018) (width 0.508) (layer F.Cu) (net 9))
 (via (at 73.5045 68.018) (size 0.508) (drill 0.3048) (layers F.Cu B.Cu) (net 9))
 (segment (start 73.5045 68.703) (end 73.5045 68.018) (width 0.508) (layer B.Cu) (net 9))
 (segment (start 74.4635 69.662) (end 73.5045 68.703) (width 0.508) (layer B.Cu) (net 9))
 (segment (start 77.4545 66.557) (end 77.4545 66.684) (width 0.508) (layer F.Cu) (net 9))
 (segment (start 77.4545 64.238) (end 77.4545 66.557) (width 0.508) (layer F.Cu) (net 9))
 (segment (start 77.4545 66.684) (end 78.1835 67.413) (width 0.508) (layer F.Cu) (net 9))
 (segment (start 78.1835 67.413) (end 78.1835 68.048) (width 0.508) (layer F.Cu) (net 9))
 (segment (start 78.1835 68.048) (end 78.1835 68.048) (width 0.508) (layer F.Cu) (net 9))
 (via (at 78.1835 68.048) (size 0.508) (drill 0.3048) (layers F.Cu B.Cu) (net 9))
 (segment (start 75.8075 69.662) (end 77.4585 69.662) (width 0.508) (layer B.Cu) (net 9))
 (segment (start 75.8075 69.662) (end 74.4635 69.662) (width 0.508) (layer B.Cu) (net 9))
 (segment (start 76.5695 69.662) (end 75.8075 69.662) (width 0.508) (layer B.Cu) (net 9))
 (segment (start 78.1835 68.937) (end 78.1835 68.048) (width 0.508) (layer B.Cu) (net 9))
 (segment (start 77.4585 69.662) (end 78.1835 68.937) (width 0.508) (layer B.Cu) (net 9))
 (segment (start 79.3245 59.143) (end 70.6845 59.143) (width 0.508) (layer F.Cu) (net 3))
 (segment (start 70.6845 59.143) (end 70.6845 63.323) (width 0.508) (layer F.Cu) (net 3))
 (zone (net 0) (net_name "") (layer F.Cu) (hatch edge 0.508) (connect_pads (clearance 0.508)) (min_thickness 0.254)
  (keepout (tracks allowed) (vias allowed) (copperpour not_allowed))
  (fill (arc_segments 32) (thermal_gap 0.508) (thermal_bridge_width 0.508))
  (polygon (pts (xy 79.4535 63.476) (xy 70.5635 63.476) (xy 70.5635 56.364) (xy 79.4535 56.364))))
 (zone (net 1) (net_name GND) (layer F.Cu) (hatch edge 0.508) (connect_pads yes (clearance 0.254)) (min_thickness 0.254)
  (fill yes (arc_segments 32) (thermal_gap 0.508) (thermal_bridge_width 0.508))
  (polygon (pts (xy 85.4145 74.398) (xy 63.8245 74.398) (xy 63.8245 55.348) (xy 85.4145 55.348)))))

